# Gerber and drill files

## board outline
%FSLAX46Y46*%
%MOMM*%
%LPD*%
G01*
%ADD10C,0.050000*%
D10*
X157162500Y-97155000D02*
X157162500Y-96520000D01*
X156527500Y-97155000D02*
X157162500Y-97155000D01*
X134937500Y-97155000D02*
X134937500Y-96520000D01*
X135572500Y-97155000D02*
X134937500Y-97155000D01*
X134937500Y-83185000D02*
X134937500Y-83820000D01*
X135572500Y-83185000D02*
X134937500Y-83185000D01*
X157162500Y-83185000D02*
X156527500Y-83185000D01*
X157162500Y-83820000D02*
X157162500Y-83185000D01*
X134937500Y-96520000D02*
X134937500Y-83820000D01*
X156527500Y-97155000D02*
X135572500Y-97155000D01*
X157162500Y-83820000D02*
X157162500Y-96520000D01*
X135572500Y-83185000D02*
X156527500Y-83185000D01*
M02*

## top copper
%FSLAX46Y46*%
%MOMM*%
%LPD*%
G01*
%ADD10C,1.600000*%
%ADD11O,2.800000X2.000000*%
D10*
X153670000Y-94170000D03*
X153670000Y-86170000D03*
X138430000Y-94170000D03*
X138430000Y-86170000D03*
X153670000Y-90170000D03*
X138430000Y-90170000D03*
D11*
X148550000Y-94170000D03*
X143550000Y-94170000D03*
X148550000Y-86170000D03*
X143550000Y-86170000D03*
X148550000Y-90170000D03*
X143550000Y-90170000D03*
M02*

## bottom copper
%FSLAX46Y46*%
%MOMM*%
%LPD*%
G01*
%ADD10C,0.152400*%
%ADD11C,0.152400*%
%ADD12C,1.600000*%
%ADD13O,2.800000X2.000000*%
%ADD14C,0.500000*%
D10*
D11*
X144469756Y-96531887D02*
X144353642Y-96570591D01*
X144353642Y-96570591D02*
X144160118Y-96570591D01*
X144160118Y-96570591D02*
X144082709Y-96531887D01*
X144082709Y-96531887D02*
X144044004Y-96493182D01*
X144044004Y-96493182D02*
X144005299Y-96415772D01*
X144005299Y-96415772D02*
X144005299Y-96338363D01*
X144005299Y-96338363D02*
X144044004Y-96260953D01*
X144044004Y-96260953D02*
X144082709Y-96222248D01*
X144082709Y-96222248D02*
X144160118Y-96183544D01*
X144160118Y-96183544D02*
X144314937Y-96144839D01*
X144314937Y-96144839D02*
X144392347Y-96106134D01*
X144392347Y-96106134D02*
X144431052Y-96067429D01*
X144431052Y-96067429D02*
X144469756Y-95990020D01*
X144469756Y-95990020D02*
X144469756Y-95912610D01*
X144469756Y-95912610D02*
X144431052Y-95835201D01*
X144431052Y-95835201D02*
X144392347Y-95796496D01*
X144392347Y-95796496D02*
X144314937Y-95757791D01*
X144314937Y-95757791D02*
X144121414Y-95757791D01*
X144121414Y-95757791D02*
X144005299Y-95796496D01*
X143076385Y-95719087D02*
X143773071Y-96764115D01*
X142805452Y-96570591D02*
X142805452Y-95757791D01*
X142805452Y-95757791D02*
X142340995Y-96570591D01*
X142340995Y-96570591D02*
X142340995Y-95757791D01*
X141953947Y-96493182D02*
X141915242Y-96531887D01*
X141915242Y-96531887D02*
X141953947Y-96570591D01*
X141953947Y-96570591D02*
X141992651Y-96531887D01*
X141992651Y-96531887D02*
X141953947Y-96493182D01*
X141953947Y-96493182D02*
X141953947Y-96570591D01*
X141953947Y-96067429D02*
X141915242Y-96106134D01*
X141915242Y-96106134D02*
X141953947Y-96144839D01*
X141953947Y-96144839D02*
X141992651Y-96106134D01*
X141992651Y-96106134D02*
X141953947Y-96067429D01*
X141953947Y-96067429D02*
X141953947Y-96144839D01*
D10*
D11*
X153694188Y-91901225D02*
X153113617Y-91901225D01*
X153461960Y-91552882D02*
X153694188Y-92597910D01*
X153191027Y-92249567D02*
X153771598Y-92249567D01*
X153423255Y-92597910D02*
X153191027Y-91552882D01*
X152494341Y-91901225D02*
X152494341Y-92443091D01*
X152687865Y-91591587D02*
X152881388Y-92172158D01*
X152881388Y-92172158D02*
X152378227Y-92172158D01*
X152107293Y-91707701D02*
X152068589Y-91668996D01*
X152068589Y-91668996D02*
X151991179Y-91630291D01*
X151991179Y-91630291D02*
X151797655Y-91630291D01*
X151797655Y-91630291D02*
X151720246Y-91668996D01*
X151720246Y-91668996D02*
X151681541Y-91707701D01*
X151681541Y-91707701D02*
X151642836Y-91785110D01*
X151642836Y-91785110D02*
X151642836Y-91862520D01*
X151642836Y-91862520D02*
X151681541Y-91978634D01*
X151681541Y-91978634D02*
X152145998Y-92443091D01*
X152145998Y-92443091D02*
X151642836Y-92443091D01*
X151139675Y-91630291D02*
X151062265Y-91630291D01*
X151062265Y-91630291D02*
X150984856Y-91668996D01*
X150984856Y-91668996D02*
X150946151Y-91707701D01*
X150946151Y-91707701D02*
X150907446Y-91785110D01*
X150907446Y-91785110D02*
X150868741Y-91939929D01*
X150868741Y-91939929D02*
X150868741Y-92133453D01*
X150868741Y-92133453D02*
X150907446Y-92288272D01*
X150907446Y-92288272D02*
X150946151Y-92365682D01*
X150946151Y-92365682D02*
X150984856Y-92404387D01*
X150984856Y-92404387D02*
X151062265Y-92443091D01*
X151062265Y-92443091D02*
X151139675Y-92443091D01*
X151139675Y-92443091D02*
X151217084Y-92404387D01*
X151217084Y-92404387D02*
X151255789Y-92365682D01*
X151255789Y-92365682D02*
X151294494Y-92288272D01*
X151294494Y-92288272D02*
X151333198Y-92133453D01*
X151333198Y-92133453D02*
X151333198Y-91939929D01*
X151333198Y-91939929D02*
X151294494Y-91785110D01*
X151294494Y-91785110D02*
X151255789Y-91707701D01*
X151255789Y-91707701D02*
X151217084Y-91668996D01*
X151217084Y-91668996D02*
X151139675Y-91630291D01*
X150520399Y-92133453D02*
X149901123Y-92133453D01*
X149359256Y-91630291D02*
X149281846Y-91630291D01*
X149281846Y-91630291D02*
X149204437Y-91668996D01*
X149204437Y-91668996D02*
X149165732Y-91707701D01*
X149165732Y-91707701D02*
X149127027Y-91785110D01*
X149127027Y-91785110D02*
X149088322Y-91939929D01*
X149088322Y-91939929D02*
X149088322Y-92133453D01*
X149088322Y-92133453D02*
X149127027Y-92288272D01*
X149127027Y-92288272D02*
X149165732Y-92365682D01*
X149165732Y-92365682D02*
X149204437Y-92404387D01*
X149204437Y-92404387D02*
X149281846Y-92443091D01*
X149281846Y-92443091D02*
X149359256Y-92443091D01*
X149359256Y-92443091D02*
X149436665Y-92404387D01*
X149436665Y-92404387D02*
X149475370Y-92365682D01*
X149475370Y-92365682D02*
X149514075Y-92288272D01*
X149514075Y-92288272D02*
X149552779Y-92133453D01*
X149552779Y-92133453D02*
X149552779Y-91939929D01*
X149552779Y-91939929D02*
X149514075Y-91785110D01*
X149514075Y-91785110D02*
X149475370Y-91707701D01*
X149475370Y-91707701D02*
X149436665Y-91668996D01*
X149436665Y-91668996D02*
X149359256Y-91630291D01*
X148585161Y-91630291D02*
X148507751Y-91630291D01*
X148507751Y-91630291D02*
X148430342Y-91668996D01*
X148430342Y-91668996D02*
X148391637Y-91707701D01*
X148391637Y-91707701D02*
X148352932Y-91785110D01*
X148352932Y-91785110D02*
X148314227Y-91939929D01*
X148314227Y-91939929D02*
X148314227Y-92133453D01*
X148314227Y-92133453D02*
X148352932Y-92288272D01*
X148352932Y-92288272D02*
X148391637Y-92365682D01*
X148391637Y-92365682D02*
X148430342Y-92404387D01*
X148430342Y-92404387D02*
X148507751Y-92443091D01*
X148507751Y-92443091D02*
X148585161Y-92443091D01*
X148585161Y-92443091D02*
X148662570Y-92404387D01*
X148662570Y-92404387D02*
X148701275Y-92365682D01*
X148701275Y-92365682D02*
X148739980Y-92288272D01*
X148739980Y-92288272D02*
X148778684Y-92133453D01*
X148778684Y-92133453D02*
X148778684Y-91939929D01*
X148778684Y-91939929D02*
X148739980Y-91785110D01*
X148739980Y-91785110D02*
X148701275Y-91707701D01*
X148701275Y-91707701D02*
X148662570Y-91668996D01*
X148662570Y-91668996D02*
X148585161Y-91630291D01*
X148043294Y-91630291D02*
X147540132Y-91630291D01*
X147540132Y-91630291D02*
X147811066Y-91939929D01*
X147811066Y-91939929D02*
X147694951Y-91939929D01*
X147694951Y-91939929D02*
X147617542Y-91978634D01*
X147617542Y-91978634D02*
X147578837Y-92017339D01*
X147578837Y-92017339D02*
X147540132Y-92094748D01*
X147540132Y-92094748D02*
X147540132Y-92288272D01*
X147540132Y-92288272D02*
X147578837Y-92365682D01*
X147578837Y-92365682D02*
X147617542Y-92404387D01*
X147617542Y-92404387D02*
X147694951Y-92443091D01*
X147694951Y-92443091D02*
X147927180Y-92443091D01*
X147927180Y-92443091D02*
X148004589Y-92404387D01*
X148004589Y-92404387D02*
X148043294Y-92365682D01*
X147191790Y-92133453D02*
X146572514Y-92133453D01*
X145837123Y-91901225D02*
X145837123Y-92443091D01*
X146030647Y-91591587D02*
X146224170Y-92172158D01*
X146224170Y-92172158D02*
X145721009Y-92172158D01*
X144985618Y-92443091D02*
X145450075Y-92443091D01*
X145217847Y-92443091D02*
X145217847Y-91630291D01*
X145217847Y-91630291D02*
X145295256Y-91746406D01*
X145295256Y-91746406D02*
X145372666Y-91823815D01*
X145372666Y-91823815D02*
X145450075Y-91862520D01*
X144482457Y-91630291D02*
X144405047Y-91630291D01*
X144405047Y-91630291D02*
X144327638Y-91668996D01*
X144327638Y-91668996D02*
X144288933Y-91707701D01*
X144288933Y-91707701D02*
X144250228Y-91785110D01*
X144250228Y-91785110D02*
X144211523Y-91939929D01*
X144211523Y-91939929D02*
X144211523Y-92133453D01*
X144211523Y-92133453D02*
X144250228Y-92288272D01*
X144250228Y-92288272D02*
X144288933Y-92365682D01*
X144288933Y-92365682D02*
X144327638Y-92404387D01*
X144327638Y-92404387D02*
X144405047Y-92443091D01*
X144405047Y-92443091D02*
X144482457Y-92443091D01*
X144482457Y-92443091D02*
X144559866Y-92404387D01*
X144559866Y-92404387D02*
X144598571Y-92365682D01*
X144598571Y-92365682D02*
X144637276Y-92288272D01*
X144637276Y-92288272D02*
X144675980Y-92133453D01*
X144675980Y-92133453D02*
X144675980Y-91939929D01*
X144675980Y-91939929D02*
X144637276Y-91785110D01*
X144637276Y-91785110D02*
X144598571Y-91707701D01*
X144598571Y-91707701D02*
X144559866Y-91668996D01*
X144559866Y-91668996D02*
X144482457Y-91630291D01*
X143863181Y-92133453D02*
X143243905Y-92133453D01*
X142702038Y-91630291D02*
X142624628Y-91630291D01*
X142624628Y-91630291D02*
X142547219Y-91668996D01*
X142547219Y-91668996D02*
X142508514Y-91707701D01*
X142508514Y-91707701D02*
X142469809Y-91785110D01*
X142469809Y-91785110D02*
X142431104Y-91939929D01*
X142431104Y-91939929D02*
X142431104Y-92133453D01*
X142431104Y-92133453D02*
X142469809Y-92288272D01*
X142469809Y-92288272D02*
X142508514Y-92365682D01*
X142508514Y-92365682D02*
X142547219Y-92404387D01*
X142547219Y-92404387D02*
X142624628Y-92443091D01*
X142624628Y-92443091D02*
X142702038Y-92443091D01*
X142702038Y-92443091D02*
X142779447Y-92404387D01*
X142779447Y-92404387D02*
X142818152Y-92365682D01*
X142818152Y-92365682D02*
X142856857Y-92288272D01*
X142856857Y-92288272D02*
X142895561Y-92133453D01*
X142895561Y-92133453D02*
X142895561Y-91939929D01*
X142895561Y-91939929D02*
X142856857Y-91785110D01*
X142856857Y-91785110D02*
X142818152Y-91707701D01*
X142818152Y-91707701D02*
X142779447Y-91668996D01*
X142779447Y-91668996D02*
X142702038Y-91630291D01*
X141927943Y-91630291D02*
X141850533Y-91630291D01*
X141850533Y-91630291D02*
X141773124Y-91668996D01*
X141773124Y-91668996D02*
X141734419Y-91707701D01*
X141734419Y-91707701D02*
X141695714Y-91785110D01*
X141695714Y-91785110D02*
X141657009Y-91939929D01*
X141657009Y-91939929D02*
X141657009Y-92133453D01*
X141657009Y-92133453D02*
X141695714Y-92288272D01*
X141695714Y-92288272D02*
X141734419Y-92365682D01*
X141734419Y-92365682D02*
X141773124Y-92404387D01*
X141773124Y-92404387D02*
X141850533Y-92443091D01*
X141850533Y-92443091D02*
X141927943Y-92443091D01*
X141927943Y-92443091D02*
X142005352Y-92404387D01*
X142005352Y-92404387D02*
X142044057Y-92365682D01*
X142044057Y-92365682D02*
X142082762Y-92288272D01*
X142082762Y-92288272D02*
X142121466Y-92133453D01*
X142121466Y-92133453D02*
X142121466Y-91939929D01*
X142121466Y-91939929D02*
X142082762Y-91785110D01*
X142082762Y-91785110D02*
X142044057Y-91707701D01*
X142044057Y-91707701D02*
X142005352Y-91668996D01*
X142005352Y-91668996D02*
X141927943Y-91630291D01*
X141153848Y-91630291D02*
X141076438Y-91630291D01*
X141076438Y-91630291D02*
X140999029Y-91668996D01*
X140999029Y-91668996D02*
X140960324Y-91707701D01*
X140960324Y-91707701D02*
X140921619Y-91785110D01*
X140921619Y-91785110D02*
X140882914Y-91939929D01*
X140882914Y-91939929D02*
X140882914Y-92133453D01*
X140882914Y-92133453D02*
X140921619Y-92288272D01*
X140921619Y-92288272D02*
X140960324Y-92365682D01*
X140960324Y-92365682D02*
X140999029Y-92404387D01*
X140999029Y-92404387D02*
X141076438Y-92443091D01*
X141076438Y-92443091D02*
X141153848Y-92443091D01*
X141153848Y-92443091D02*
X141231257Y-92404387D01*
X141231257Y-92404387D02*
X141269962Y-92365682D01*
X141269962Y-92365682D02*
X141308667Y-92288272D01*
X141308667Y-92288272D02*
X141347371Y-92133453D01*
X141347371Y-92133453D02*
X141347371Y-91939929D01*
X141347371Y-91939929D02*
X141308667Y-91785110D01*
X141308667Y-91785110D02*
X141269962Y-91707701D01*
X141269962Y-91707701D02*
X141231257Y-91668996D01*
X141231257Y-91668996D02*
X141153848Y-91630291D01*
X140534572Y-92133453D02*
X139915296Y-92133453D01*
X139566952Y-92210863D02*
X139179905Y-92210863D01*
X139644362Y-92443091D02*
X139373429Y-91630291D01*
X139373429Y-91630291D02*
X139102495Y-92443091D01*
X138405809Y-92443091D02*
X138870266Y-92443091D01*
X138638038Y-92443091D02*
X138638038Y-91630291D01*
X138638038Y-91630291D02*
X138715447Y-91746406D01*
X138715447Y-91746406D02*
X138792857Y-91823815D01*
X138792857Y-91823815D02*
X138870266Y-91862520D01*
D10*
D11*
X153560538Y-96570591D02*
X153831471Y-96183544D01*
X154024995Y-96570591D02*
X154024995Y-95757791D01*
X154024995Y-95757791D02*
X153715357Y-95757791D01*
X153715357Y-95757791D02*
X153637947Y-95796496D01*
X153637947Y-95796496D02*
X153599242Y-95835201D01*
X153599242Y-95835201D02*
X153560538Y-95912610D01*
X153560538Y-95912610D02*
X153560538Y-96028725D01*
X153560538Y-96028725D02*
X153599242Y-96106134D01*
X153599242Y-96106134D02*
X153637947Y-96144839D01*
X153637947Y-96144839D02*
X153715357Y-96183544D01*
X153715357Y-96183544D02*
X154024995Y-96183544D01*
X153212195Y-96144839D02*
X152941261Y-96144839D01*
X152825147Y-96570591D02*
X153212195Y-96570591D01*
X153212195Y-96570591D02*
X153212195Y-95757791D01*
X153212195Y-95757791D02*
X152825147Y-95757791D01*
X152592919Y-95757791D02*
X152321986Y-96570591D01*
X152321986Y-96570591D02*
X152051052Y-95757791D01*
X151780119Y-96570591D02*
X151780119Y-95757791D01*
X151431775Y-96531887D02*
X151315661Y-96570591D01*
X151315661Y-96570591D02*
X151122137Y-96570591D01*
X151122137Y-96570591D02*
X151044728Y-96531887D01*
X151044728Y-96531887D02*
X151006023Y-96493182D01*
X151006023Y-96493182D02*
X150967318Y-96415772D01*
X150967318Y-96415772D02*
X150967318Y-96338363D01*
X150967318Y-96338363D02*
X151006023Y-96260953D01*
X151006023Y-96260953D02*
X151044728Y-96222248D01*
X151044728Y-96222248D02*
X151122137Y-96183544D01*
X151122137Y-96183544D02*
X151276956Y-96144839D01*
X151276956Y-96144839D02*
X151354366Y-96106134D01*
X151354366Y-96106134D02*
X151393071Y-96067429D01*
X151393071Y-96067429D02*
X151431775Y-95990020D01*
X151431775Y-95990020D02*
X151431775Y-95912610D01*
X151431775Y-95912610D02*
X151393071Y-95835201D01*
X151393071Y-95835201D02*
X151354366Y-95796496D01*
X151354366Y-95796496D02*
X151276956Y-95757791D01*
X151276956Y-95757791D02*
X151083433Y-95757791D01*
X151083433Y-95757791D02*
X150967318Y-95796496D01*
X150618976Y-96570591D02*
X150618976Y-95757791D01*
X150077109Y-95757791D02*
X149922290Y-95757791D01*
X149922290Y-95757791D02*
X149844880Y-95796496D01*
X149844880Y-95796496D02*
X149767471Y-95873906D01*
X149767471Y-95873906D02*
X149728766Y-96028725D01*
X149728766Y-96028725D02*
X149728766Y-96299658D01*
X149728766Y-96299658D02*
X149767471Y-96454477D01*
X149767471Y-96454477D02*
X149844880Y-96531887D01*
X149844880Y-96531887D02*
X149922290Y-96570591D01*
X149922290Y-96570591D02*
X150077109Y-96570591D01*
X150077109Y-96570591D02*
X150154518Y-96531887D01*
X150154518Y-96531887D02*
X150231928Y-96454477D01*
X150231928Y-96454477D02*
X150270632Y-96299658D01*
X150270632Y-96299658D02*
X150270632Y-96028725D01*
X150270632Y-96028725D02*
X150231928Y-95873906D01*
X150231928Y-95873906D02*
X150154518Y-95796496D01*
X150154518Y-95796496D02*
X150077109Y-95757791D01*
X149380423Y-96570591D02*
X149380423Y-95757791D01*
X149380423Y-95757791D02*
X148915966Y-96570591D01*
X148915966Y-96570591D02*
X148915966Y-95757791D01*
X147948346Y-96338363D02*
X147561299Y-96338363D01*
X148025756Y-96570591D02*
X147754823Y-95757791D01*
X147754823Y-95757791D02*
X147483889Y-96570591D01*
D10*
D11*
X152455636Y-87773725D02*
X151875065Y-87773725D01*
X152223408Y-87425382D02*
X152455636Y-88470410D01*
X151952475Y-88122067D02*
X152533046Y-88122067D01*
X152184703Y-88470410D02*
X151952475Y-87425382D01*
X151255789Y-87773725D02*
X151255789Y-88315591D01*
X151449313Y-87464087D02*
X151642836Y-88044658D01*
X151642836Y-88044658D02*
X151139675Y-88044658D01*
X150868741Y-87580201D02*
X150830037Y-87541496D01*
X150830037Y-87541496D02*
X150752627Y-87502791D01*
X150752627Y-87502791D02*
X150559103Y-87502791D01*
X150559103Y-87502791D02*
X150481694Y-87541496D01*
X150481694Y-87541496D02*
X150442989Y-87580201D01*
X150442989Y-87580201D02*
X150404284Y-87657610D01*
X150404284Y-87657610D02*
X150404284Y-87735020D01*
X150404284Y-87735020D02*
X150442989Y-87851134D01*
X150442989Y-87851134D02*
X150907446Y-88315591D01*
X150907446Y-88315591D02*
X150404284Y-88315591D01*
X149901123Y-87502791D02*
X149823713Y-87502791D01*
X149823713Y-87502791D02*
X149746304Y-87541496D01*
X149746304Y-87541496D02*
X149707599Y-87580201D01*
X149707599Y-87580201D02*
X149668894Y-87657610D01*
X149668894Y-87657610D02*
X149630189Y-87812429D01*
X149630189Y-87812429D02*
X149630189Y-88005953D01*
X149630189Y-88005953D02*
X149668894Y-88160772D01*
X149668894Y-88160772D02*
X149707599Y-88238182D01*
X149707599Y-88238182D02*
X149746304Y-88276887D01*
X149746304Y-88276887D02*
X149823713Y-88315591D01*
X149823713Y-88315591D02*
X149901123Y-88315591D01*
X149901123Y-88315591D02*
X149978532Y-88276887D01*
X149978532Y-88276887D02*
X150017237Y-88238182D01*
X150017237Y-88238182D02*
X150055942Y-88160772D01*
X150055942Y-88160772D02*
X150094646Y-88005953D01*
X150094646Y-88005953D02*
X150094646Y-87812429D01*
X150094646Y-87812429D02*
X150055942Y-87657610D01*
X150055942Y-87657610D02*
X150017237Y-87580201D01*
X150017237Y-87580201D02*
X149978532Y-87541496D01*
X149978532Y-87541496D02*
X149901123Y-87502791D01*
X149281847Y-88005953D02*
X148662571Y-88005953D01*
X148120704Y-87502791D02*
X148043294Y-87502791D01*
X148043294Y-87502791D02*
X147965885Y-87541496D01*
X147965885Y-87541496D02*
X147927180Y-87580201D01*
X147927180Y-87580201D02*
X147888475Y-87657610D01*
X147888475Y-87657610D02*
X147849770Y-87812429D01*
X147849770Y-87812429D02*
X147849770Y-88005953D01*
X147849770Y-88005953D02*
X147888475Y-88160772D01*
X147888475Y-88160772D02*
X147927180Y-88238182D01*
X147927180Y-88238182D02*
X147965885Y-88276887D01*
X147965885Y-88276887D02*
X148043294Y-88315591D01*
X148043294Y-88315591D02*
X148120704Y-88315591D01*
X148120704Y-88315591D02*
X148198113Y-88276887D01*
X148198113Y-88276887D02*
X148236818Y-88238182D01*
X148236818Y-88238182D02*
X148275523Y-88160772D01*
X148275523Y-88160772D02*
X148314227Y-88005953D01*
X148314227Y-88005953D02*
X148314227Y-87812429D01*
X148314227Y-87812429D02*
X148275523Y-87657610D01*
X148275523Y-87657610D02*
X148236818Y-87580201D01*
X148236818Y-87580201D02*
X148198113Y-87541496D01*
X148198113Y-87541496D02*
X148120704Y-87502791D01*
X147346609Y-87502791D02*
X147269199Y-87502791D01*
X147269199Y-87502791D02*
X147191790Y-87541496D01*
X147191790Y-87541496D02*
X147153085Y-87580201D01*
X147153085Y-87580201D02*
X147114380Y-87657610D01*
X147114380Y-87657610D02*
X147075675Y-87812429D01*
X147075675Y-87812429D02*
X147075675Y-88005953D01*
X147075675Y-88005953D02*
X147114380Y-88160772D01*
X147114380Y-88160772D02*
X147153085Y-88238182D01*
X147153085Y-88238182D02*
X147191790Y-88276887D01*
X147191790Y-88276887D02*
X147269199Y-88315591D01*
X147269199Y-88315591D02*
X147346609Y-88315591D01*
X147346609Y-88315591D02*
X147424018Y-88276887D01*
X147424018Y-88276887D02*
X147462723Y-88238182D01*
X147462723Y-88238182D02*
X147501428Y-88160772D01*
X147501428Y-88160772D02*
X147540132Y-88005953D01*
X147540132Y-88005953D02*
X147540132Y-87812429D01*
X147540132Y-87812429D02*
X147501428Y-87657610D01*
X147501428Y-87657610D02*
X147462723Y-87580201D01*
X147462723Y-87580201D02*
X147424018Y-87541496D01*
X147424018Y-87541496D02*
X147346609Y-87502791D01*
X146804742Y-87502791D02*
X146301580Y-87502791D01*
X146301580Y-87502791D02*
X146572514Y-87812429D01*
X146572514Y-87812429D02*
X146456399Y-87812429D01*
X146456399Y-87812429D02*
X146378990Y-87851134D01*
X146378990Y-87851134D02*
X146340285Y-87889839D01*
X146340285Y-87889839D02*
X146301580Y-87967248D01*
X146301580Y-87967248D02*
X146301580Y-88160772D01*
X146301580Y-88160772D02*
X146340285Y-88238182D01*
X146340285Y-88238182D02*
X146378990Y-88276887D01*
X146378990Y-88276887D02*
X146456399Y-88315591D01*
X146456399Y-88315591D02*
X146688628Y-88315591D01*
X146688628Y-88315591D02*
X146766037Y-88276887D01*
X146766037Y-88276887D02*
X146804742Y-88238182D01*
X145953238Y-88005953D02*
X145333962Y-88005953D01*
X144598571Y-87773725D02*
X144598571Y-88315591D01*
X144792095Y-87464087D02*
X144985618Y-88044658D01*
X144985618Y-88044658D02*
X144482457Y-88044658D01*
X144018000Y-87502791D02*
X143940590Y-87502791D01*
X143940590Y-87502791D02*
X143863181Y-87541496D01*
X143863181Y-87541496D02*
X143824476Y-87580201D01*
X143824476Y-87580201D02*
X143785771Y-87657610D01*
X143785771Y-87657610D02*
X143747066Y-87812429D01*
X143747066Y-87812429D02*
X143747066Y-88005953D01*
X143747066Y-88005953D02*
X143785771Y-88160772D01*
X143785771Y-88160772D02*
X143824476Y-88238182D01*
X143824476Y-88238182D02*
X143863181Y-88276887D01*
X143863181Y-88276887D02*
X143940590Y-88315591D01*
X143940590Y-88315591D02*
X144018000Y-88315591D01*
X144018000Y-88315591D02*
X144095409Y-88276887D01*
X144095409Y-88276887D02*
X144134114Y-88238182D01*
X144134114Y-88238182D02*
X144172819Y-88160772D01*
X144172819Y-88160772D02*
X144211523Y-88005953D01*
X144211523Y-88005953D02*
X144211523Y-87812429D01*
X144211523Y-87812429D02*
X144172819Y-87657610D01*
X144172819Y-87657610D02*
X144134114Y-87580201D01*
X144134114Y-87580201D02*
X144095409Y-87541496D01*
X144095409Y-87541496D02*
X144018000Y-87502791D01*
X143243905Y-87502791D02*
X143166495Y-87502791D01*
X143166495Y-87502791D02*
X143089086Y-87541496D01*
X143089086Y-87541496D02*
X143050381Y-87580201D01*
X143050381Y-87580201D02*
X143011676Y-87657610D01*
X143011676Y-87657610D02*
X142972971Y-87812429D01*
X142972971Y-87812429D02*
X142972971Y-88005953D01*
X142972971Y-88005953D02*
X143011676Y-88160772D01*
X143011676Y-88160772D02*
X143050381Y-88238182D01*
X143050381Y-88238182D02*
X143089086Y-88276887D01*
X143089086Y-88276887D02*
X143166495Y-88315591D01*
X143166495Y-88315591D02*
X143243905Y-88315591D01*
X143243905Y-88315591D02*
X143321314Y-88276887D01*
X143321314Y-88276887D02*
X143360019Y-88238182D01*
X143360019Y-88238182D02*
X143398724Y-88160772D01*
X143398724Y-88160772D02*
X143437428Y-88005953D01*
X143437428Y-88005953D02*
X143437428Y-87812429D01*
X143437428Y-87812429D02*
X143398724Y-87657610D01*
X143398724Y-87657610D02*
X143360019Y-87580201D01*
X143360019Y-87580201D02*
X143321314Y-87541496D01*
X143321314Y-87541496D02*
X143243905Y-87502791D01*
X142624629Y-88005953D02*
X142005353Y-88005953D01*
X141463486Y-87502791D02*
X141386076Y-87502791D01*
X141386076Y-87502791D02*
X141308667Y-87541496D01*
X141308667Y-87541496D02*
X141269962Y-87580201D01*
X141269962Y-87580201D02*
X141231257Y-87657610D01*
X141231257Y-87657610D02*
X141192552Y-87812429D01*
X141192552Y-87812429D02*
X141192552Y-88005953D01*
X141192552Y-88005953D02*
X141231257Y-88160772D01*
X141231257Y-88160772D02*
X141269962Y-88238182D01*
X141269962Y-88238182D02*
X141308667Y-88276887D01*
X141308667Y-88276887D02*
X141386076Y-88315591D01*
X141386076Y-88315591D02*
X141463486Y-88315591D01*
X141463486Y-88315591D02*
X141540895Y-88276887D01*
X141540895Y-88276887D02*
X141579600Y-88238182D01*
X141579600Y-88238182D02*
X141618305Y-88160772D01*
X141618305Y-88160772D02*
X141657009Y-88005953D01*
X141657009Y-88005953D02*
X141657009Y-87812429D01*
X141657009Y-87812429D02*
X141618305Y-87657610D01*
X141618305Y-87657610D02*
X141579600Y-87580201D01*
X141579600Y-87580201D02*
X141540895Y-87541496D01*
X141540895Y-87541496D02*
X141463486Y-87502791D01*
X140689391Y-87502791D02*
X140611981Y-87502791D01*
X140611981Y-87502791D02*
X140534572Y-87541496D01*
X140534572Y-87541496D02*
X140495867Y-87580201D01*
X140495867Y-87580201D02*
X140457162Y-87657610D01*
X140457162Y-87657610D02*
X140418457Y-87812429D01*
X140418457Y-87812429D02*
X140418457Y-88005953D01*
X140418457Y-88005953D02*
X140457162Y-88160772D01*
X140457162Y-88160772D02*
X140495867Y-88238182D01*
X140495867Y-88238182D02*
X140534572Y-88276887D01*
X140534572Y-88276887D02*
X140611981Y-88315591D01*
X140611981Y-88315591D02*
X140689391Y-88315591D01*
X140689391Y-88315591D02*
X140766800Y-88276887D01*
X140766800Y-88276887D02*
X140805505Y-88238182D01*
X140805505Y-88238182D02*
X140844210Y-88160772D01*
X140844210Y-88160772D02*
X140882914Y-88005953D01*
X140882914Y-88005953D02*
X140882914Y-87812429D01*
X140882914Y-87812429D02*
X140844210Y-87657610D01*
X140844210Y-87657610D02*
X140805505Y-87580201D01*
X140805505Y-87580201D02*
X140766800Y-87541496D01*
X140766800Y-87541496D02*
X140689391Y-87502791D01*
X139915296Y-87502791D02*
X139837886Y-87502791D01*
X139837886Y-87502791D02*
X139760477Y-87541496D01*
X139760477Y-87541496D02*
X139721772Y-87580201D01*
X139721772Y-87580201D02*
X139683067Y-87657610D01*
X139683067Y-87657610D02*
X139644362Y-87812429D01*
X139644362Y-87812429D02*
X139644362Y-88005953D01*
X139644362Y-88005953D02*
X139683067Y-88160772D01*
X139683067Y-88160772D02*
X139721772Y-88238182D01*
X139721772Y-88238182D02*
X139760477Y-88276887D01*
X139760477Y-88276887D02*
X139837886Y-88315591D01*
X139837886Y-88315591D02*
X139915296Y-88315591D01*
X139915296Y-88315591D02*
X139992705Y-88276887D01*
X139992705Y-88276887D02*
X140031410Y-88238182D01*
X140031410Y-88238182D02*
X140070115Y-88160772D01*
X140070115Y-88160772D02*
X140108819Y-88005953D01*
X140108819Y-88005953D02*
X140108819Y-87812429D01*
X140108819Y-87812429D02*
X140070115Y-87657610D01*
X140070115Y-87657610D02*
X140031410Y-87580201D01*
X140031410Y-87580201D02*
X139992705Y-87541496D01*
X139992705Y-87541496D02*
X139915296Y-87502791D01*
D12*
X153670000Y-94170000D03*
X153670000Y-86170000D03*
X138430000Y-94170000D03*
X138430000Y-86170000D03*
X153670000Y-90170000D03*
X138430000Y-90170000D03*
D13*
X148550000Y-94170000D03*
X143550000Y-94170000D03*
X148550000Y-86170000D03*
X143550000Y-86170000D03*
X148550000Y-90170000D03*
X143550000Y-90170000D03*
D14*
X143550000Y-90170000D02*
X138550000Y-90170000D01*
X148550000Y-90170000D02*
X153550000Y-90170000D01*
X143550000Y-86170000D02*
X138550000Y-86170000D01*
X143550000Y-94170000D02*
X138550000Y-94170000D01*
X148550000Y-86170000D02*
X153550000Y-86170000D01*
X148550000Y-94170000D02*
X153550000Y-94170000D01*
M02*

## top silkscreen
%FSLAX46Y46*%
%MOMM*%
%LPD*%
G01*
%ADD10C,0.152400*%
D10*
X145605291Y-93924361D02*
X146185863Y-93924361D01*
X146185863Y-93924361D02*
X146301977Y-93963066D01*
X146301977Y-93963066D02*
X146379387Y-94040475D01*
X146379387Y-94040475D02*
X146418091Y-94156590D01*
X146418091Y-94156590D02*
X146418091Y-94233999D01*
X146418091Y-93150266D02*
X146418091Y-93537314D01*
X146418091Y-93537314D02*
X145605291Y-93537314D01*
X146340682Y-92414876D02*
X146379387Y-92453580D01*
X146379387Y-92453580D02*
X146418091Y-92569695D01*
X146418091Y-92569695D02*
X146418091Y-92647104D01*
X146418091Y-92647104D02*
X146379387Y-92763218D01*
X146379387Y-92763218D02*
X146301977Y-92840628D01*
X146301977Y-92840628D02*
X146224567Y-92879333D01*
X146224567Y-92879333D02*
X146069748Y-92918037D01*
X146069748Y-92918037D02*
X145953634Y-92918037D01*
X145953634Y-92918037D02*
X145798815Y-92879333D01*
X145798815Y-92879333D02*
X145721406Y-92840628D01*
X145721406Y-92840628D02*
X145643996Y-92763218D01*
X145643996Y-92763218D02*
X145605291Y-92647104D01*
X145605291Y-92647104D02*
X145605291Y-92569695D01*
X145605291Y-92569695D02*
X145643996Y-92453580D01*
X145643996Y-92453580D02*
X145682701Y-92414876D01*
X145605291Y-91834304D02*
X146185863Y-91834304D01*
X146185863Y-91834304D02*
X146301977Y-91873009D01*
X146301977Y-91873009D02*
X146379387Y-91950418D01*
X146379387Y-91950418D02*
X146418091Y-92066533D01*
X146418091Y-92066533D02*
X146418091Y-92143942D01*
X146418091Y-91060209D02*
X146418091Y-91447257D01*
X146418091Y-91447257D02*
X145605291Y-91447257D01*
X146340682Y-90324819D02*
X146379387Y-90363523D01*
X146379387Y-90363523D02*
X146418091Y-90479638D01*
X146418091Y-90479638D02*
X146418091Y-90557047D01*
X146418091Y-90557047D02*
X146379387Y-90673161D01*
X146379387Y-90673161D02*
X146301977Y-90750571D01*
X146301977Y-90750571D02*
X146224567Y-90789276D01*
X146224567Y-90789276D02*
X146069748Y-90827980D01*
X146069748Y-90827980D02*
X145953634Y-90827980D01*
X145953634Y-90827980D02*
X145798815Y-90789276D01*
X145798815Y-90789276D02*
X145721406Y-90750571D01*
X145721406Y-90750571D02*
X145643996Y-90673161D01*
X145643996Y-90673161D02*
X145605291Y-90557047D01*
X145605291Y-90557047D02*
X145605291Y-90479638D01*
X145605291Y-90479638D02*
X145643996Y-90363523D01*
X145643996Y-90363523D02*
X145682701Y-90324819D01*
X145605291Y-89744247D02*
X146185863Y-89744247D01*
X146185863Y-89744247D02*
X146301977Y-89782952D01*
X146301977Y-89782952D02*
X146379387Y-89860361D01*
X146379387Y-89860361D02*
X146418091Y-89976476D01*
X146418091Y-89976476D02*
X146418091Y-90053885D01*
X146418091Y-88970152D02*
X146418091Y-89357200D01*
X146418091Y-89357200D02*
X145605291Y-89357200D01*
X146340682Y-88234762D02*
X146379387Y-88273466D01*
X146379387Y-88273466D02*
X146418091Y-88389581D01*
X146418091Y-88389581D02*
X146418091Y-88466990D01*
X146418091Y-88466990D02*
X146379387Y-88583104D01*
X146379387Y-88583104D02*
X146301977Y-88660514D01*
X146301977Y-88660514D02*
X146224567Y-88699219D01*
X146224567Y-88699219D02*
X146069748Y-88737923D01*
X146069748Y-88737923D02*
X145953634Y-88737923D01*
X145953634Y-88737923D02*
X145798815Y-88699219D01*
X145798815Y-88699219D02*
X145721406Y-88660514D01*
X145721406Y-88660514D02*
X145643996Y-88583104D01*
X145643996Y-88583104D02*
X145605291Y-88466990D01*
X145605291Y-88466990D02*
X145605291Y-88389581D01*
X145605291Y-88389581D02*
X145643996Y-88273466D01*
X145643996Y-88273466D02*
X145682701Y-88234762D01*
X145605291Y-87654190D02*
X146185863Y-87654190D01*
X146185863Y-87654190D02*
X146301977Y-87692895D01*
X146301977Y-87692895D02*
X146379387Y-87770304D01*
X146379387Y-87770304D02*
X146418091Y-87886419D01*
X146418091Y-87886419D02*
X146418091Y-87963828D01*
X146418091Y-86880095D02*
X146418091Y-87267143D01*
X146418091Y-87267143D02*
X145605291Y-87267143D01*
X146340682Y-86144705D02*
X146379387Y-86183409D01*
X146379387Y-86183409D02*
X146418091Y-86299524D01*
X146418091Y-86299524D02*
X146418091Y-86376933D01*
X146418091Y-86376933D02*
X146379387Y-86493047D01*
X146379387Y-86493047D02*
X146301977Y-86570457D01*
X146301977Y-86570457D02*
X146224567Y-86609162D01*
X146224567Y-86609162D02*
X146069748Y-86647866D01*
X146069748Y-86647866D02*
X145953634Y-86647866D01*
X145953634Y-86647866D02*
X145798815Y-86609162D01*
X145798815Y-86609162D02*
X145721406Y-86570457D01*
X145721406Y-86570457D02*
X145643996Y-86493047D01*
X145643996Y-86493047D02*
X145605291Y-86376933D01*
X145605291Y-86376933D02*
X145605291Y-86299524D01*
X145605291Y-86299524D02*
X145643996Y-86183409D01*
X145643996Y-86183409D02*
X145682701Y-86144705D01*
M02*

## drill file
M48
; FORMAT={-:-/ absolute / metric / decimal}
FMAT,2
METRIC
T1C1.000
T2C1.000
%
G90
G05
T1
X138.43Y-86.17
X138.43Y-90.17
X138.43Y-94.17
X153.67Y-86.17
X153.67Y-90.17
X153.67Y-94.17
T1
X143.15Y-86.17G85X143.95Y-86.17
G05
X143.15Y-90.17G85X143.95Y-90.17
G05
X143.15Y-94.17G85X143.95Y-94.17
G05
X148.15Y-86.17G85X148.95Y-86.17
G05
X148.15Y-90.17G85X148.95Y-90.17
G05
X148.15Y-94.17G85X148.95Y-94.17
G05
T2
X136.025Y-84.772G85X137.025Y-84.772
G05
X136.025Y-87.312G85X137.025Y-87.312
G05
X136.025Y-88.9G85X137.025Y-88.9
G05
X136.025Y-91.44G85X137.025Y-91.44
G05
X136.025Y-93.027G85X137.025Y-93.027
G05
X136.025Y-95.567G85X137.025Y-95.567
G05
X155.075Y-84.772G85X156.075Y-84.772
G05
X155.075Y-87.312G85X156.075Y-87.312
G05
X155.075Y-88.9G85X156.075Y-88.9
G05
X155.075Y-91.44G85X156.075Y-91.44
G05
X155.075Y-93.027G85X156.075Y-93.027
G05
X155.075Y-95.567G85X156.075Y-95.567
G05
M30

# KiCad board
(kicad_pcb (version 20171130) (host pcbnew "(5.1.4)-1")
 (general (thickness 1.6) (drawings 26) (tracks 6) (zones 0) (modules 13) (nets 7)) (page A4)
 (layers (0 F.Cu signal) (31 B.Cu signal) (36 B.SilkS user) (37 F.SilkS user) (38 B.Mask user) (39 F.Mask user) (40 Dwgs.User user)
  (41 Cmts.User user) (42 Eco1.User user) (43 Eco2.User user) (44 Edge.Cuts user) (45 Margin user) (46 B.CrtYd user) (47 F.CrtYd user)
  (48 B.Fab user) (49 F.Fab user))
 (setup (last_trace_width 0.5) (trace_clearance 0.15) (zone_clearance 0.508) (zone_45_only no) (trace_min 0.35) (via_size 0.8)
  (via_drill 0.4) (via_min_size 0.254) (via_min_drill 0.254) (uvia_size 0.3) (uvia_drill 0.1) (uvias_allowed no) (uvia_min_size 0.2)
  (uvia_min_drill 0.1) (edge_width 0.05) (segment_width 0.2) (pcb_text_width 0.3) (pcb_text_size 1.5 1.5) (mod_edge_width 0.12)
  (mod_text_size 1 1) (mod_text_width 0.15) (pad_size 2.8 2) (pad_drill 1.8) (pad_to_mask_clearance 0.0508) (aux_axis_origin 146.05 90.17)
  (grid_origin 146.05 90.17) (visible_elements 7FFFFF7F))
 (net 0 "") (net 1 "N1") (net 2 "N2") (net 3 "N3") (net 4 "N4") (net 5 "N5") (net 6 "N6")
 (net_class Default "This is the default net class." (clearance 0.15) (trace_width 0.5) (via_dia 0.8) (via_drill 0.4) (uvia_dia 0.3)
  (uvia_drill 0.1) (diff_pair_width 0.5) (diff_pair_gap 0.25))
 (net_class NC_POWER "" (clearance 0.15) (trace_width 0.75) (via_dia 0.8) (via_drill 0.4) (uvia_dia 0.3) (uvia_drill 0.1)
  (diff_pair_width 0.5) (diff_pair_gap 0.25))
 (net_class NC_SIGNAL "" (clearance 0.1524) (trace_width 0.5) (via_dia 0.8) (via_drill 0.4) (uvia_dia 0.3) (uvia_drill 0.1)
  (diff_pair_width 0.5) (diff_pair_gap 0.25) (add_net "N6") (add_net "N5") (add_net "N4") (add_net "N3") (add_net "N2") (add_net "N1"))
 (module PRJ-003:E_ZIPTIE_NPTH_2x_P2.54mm (layer F.Cu) (at 136.525 86.0425 90)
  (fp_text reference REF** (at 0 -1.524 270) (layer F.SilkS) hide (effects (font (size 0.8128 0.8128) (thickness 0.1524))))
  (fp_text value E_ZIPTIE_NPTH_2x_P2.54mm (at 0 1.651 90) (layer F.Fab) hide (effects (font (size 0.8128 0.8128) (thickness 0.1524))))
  (pad "" np_thru_hole oval (at -1.27 0 90) (size 1 2) (drill oval 1 2) (layers *.Cu *.Mask))
  (pad "" np_thru_hole oval (at 1.27 0 90) (size 1 2) (drill oval 1 2) (layers *.Cu *.Mask)))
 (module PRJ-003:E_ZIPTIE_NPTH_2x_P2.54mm (layer F.Cu) (at 136.525 90.17 90)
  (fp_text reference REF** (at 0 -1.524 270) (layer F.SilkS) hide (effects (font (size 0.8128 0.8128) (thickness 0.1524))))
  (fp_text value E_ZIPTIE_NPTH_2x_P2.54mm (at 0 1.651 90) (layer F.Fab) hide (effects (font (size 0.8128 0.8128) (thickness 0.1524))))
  (pad "" np_thru_hole oval (at 1.27 0 90) (size 1 2) (drill oval 1 2) (layers *.Cu *.Mask))
  (pad "" np_thru_hole oval (at -1.27 0 90) (size 1 2) (drill oval 1 2) (layers *.Cu *.Mask)))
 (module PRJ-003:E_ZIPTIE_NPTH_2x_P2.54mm (layer F.Cu) (at 136.525 94.2975 90)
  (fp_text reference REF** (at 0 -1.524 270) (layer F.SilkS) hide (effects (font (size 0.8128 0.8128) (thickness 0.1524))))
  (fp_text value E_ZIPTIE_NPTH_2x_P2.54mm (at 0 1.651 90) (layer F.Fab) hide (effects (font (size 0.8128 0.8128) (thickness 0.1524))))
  (pad "" np_thru_hole oval (at -1.27 0 90) (size 1 2) (drill oval 1 2) (layers *.Cu *.Mask))
  (pad "" np_thru_hole oval (at 1.27 0 90) (size 1 2) (drill oval 1 2) (layers *.Cu *.Mask)))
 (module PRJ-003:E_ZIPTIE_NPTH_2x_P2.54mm (layer F.Cu) (at 155.575 94.2975 90)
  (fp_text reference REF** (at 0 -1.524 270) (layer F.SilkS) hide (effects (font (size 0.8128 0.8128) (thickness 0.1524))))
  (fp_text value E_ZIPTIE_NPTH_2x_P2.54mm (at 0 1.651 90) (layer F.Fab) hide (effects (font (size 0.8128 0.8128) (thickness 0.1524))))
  (pad "" np_thru_hole oval (at 1.27 0 90) (size 1 2) (drill oval 1 2) (layers *.Cu *.Mask))
  (pad "" np_thru_hole oval (at -1.27 0 90) (size 1 2) (drill oval 1 2) (layers *.Cu *.Mask)))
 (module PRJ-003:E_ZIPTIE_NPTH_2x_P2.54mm (layer F.Cu) (at 155.575 90.17 90)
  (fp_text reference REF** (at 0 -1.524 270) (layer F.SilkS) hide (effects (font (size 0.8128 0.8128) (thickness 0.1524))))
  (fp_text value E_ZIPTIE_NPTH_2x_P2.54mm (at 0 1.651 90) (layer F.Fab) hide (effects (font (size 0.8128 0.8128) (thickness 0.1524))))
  (pad "" np_thru_hole oval (at -1.27 0 90) (size 1 2) (drill oval 1 2) (layers *.Cu *.Mask))
  (pad "" np_thru_hole oval (at 1.27 0 90) (size 1 2) (drill oval 1 2) (layers *.Cu *.Mask)))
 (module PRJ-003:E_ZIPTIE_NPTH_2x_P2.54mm (layer F.Cu) (at 155.575 86.0425 90)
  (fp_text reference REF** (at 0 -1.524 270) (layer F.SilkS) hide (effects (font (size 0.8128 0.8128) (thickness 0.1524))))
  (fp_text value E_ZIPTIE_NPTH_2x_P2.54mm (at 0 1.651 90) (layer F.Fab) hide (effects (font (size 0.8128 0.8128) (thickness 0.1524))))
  (pad "" np_thru_hole oval (at 1.27 0 90) (size 1 2) (drill oval 1 2) (layers *.Cu *.Mask))
  (pad "" np_thru_hole oval (at -1.27 0 90) (size 1 2) (drill oval 1 2) (layers *.Cu *.Mask)))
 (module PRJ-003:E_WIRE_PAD (layer F.Cu) (at 153.67 94.17)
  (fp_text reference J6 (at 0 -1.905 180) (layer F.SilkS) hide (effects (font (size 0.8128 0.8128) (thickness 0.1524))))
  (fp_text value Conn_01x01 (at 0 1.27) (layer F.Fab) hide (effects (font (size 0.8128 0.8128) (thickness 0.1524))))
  (pad "" connect circle (at 0 0) (size 1 1) (layers F.Mask))
  (pad 1 thru_hole circle (at 0 0) (size 1.6 1.6) (drill 1) (layers B.Cu B.Mask) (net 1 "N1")))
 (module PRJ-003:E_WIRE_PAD (layer F.Cu) (at 153.67 86.17)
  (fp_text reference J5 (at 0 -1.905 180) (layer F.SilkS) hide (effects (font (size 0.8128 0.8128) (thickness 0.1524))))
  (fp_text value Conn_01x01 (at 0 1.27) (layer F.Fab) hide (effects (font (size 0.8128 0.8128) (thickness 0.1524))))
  (pad "" connect circle (at 0 0) (size 1 1) (layers F.Mask))
  (pad 1 thru_hole circle (at 0 0) (size 1.6 1.6) (drill 1) (layers B.Cu B.Mask) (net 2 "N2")))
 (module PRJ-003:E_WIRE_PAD (layer F.Cu) (at 138.43 94.17)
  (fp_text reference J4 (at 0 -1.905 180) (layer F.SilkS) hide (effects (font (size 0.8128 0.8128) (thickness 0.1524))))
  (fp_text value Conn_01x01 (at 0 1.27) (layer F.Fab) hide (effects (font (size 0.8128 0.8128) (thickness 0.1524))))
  (pad "" connect circle (at 0 0) (size 1 1) (layers F.Mask))
  (pad 1 thru_hole circle (at 0 0) (size 1.6 1.6) (drill 1) (layers B.Cu B.Mask) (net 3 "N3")))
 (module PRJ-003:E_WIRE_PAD (layer F.Cu) (at 138.43 86.17)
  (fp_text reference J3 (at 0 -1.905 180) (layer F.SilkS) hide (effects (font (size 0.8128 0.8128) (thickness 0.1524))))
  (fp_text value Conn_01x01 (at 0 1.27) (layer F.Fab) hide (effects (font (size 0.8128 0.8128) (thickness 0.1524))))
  (pad "" connect circle (at 0 0) (size 1 1) (layers F.Mask))
  (pad 1 thru_hole circle (at 0 0) (size 1.6 1.6) (drill 1) (layers B.Cu B.Mask) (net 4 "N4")))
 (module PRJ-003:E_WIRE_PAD (layer F.Cu) (at 153.67 90.17)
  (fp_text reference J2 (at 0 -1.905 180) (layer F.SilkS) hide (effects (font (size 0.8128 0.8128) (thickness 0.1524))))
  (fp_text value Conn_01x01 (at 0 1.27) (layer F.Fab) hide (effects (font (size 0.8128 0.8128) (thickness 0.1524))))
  (pad "" connect circle (at 0 0) (size 1 1) (layers F.Mask))
  (pad 1 thru_hole circle (at 0 0) (size 1.6 1.6) (drill 1) (layers B.Cu B.Mask) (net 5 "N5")))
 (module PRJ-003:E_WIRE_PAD (layer F.Cu) (at 138.43 90.17)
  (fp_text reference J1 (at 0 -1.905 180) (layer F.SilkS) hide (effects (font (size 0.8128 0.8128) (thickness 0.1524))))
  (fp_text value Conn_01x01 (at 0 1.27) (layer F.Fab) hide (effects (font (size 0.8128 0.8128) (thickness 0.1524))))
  (pad "" connect circle (at 0 0) (size 1 1) (layers F.Mask))
  (pad 1 thru_hole circle (at 0 0) (size 1.6 1.6) (drill 1) (layers B.Cu B.Mask) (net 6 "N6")))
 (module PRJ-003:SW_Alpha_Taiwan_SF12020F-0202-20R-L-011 (layer F.Cu) (at 146.05 90.17)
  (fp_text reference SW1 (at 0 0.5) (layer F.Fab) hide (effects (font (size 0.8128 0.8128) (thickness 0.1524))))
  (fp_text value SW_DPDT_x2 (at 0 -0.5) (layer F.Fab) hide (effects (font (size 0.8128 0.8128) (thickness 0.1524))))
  (pad 6 thru_hole oval (at 2.5 4) (size 2.8 2) (drill oval 1.8 1) (layers *.Cu *.Mask) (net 1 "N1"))
  (pad 3 thru_hole oval (at -2.5 4) (size 2.8 2) (drill oval 1.8 1) (layers *.Cu *.Mask) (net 3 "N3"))
  (pad 4 thru_hole oval (at 2.5 -4) (size 2.8 2) (drill oval 1.8 1) (layers *.Cu *.Mask) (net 2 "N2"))
  (pad 1 thru_hole oval (at -2.5 -4) (size 2.8 2) (drill oval 1.8 1) (layers *.Cu *.Mask) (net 4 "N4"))
  (pad 5 thru_hole oval (at 2.5 0) (size 2.8 2) (drill oval 1.8 1) (layers *.Cu *.Mask) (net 5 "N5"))
  (pad 2 thru_hole oval (at -2.5 0) (size 2.8 2) (drill oval 1.8 1) (layers *.Cu *.Mask) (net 6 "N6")))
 (gr_line (start 157.1625 97.155) (end 157.1625 96.52) (layer Edge.Cuts) (width 0.05))
 (gr_line (start 156.5275 97.155) (end 157.1625 97.155) (layer Edge.Cuts) (width 0.05))
 (gr_line (start 134.9375 97.155) (end 134.9375 96.52) (layer Edge.Cuts) (width 0.05))
 (gr_line (start 135.5725 97.155) (end 134.9375 97.155) (layer Edge.Cuts) (width 0.05))
 (gr_line (start 134.9375 83.185) (end 134.9375 83.82) (layer Edge.Cuts) (width 0.05))
 (gr_line (start 135.5725 83.185) (end 134.9375 83.185) (layer Edge.Cuts) (width 0.05))
 (gr_line (start 157.1625 83.185) (end 156.5275 83.185) (layer Edge.Cuts) (width 0.05))
 (gr_line (start 157.1625 83.82) (end 157.1625 83.185) (layer Edge.Cuts) (width 0.05))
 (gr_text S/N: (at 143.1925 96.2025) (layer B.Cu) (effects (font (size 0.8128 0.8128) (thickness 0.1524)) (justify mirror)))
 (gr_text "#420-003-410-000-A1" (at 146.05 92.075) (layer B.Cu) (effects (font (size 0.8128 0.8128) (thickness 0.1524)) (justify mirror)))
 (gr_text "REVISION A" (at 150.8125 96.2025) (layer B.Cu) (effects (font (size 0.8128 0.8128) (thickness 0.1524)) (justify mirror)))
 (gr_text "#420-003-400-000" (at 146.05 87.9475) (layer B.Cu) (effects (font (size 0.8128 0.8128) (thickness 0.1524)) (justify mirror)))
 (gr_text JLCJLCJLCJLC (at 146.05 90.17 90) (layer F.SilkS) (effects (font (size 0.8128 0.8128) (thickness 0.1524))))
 (gr_line (start 134.9375 96.52) (end 134.9375 83.82) (layer Edge.Cuts) (width 0.05))
 (gr_line (start 156.5275 97.155) (end 135.5725 97.155) (layer Edge.Cuts) (width 0.05))
 (gr_line (start 157.1625 83.82) (end 157.1625 96.52) (layer Edge.Cuts) (width 0.05))
 (gr_line (start 135.5725 83.185) (end 156.5275 83.185) (layer Edge.Cuts) (width 0.05))
 (segment (start 143.55 90.17) (end 138.55 90.17) (width 0.5) (layer B.Cu) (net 6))
 (segment (start 148.55 90.17) (end 153.55 90.17) (width 0.5) (layer B.Cu) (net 5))
 (segment (start 143.55 86.17) (end 138.55 86.17) (width 0.5) (layer B.Cu) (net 4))
 (segment (start 143.55 94.17) (end 138.55 94.17) (width 0.5) (layer B.Cu) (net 3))
 (segment (start 148.55 86.17) (end 153.55 86.17) (width 0.5) (layer B.Cu) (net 2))
 (segment (start 148.55 94.17) (end 153.55 94.17) (width 0.5) (layer B.Cu) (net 1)))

